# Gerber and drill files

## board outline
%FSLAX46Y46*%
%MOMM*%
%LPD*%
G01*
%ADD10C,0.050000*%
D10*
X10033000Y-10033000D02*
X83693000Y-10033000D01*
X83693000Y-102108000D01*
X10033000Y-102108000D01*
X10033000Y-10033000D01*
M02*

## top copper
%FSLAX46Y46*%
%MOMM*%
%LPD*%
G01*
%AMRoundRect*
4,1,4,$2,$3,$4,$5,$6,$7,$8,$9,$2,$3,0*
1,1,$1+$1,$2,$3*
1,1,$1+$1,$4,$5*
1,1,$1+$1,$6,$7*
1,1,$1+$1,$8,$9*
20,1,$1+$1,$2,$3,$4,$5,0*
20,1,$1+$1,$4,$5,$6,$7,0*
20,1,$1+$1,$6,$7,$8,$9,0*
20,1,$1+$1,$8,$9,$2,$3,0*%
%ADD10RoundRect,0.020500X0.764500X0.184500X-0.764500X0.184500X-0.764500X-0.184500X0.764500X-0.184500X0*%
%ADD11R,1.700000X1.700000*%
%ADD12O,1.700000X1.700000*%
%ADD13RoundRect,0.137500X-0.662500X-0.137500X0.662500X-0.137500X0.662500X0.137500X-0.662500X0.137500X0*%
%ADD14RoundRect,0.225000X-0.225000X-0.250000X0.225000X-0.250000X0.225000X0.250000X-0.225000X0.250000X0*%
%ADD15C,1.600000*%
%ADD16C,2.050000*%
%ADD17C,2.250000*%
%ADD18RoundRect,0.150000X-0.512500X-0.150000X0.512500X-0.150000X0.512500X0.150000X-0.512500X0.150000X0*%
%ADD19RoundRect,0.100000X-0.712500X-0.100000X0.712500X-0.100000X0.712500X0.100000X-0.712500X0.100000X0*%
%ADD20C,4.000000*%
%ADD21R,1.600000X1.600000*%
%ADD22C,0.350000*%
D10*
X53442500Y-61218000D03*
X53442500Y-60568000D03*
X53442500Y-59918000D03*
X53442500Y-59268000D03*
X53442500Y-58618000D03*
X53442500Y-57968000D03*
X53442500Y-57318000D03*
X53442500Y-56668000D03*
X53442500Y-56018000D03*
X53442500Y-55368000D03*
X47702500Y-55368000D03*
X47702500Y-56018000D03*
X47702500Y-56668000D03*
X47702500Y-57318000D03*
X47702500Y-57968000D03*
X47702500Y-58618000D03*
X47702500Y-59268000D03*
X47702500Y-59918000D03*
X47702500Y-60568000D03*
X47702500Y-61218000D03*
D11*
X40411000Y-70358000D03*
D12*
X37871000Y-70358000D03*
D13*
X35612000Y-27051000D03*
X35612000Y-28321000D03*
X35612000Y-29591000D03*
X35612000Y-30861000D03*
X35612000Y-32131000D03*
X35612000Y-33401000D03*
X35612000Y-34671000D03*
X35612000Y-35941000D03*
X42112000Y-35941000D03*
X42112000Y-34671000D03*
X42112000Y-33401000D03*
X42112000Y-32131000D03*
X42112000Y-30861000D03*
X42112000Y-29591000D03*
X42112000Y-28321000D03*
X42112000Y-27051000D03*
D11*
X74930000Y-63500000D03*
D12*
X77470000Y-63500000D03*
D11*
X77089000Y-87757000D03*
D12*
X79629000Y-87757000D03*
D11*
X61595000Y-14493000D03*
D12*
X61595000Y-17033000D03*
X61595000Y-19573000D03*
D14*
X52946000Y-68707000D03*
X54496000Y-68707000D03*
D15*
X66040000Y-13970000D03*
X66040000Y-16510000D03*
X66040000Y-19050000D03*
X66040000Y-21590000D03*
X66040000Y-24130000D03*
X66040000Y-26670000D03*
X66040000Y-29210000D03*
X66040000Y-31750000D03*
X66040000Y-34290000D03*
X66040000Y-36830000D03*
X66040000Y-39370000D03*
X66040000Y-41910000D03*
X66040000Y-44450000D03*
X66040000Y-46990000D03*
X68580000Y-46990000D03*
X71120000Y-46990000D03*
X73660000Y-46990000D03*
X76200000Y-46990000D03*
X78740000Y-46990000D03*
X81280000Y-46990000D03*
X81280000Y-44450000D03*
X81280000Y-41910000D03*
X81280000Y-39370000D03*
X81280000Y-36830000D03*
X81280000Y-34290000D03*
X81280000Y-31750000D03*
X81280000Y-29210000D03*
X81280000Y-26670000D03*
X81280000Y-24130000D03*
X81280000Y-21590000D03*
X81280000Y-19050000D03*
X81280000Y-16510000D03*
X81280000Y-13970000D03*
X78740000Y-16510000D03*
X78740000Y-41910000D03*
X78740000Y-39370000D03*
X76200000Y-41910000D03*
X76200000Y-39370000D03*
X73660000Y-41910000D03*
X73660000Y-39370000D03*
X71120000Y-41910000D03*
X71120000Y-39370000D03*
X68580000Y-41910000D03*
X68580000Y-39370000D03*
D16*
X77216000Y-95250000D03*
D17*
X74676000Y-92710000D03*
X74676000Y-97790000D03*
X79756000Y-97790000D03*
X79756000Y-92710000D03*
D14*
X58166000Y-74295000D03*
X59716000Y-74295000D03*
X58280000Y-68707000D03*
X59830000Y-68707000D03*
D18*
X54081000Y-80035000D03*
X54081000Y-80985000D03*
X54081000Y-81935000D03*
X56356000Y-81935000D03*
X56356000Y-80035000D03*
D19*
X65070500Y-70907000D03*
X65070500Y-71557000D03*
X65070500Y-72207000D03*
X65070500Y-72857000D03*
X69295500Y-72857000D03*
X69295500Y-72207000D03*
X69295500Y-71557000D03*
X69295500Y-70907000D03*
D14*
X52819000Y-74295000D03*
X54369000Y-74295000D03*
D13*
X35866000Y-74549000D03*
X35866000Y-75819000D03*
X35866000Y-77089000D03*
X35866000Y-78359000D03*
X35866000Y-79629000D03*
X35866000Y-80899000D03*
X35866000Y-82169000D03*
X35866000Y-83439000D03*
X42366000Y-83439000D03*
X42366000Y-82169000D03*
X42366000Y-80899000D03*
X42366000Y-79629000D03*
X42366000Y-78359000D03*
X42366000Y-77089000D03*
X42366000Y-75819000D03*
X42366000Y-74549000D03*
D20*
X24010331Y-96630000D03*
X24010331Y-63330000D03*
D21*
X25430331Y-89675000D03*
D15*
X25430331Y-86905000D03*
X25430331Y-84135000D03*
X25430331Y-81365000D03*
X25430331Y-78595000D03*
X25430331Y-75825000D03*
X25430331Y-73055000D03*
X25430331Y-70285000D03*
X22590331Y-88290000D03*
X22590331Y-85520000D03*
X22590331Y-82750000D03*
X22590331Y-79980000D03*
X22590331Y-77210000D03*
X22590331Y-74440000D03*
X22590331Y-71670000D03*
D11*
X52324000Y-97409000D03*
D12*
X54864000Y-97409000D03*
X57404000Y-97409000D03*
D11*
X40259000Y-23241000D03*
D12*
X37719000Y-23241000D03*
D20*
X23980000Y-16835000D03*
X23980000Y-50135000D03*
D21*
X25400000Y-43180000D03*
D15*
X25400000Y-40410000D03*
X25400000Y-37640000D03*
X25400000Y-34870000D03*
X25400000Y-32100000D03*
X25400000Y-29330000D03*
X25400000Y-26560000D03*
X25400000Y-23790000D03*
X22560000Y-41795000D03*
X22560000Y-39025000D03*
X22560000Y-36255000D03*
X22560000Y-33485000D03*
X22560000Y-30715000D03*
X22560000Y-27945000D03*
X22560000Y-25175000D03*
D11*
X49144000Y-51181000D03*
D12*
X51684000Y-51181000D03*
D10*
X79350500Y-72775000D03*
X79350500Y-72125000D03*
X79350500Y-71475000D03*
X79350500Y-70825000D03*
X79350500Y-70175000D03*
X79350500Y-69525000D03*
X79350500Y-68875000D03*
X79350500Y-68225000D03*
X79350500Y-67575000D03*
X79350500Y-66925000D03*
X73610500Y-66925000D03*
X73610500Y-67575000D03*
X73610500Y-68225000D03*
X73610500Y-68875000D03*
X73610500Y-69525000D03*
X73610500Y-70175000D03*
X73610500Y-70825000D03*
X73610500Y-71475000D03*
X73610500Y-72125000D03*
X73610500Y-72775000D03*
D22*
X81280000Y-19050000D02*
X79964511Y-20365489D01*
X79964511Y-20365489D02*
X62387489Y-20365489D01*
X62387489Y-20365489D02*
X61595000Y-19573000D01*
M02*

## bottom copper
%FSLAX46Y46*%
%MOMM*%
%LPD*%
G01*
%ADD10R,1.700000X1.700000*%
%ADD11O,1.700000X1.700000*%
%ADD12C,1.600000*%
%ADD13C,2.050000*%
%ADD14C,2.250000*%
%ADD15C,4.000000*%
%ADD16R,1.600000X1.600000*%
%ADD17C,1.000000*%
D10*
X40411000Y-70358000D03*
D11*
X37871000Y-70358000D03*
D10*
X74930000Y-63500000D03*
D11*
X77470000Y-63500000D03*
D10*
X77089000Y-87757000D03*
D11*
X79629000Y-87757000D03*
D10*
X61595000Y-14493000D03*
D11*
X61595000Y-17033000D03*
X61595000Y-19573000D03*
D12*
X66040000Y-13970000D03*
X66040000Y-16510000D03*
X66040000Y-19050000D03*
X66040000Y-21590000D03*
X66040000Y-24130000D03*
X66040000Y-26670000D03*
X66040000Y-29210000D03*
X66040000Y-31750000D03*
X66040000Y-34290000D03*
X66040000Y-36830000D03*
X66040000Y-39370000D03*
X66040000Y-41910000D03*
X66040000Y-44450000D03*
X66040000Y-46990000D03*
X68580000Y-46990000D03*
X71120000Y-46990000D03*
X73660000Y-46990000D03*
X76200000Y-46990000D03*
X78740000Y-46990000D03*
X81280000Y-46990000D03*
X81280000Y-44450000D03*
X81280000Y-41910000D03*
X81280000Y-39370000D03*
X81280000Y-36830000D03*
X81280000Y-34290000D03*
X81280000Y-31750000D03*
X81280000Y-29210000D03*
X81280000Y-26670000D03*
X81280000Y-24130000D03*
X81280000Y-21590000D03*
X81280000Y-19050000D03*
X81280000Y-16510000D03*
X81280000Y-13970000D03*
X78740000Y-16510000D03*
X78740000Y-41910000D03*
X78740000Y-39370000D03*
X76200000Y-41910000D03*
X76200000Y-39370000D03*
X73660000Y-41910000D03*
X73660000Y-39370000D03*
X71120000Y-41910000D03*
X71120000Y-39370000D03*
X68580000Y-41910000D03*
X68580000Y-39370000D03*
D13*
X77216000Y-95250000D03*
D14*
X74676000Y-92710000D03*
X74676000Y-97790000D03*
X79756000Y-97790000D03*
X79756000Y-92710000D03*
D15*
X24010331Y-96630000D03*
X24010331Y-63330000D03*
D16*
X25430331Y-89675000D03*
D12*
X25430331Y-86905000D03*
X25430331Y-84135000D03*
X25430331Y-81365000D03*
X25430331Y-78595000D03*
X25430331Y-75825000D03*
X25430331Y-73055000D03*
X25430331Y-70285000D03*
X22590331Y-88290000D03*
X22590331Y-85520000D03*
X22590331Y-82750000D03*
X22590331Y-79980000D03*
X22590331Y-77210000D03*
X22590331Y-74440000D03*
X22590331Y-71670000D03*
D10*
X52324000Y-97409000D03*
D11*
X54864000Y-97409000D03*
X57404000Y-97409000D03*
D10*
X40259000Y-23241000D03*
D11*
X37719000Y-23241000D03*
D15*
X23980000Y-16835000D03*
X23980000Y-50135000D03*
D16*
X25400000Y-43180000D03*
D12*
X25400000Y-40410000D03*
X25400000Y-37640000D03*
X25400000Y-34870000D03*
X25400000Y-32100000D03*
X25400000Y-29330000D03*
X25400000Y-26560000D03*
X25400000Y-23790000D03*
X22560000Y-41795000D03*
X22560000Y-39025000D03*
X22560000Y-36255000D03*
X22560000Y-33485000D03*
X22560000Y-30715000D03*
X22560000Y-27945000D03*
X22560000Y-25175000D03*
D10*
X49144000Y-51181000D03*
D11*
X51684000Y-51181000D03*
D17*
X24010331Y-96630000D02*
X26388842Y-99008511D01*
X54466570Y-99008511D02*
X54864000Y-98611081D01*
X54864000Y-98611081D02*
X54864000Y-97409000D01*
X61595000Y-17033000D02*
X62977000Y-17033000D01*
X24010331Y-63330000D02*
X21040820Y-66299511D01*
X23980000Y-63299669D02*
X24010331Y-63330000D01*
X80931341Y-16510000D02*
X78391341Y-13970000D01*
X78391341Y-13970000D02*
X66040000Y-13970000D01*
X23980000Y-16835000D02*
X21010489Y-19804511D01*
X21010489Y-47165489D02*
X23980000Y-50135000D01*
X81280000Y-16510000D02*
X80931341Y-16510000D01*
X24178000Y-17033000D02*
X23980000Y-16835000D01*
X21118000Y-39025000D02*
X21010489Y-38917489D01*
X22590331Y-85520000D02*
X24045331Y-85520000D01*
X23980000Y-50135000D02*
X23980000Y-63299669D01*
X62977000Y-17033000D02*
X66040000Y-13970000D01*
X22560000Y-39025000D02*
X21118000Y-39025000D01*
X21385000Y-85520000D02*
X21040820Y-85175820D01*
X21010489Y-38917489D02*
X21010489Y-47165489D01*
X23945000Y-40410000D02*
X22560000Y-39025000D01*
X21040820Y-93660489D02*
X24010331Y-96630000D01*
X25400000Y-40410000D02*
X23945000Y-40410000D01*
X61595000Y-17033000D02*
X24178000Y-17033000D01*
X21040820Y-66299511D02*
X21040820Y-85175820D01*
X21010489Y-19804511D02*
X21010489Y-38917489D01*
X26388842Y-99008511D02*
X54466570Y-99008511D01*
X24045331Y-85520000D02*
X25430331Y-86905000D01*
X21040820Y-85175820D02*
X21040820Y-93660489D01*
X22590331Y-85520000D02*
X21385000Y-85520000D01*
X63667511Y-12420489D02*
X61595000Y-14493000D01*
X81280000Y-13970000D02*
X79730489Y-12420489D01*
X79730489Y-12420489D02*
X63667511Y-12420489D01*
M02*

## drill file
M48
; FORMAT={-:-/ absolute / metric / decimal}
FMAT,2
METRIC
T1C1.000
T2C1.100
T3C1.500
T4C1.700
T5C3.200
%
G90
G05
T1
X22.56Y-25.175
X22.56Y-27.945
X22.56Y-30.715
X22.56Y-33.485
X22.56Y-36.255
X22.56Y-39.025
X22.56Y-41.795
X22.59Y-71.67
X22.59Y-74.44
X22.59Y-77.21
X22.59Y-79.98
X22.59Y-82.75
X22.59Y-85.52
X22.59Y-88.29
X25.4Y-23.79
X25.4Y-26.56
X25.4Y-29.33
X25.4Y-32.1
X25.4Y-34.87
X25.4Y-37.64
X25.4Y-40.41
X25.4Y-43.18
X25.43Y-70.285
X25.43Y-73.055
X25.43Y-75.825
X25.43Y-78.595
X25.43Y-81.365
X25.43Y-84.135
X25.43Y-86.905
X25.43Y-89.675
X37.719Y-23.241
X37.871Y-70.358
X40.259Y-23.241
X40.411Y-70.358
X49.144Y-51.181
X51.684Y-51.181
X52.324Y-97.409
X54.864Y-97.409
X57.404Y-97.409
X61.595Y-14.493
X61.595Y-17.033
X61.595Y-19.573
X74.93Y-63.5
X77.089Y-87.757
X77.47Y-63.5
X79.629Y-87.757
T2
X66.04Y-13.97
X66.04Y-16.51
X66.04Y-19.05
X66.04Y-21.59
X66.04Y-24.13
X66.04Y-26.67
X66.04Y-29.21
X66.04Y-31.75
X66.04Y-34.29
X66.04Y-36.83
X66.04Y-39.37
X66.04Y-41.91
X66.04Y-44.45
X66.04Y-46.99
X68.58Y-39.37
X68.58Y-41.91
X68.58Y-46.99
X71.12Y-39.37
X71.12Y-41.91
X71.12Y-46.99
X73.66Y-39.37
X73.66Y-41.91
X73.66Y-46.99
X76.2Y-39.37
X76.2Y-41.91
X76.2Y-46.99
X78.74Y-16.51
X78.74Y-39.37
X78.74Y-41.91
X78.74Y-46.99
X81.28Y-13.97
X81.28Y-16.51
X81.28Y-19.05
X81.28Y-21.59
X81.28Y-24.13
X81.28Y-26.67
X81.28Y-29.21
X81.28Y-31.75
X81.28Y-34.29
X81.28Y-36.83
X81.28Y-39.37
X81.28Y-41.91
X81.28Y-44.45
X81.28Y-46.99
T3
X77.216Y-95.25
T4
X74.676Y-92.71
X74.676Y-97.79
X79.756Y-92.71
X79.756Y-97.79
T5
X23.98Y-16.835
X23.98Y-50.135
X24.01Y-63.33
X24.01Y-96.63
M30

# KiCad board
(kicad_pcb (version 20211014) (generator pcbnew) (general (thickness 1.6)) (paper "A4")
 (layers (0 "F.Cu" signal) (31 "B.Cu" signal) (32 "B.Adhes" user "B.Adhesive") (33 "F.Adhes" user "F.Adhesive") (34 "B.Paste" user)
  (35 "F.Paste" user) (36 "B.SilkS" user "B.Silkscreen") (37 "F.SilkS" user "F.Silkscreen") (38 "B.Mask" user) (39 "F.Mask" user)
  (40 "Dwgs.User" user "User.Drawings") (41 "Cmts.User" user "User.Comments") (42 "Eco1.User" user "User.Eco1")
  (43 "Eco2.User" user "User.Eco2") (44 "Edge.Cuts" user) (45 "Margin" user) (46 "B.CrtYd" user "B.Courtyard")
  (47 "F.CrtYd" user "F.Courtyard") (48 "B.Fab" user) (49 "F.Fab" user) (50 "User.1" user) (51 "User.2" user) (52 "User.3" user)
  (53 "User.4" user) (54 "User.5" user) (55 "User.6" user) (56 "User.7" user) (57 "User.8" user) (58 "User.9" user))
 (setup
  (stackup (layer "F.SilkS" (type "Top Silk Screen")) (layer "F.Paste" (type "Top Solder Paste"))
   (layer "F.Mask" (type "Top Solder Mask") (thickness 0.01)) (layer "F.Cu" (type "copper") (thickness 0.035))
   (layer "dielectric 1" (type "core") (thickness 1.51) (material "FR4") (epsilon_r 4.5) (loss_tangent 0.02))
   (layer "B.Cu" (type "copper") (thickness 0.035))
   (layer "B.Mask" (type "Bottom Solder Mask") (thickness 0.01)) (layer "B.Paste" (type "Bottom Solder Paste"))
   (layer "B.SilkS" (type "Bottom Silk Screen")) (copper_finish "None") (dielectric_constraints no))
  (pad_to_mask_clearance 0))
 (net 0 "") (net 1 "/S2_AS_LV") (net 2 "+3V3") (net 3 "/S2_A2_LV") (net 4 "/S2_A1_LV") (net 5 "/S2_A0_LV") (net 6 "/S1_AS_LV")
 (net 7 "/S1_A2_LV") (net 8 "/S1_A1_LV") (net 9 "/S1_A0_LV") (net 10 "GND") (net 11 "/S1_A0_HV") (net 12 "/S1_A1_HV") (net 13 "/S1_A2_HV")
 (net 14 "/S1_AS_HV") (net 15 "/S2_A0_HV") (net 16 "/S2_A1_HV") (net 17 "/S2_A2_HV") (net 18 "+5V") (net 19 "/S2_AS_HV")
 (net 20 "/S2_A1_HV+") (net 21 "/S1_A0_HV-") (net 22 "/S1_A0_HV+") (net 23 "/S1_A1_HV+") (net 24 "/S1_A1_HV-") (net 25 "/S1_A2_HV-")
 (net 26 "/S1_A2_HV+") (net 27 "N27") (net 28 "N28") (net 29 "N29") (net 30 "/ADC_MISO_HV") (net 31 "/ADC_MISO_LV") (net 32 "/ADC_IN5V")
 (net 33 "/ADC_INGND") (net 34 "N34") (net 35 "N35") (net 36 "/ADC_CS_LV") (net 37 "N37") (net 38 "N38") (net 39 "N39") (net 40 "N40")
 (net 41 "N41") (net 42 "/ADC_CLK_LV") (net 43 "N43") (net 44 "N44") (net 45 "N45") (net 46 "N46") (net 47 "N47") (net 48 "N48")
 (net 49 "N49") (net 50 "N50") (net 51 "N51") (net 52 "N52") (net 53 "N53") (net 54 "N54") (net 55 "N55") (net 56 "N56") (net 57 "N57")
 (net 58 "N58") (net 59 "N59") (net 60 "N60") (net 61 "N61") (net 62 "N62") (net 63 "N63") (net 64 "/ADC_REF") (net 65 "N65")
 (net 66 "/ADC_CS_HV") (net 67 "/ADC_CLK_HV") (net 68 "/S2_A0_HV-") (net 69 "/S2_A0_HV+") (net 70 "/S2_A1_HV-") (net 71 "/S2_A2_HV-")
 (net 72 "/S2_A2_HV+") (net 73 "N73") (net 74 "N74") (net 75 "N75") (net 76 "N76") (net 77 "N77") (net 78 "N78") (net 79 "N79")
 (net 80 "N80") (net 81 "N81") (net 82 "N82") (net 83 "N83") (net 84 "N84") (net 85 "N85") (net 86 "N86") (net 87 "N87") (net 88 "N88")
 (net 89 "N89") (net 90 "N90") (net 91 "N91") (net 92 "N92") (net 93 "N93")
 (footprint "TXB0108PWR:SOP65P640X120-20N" (layer "F.Cu") (at 50.5725 58.293 180)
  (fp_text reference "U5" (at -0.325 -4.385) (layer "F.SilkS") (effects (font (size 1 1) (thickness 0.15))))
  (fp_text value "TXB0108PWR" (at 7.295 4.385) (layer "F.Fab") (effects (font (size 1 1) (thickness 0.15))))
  (pad "1" smd roundrect locked (at -2.87 -2.925 180) (size 1.57 0.41) (layers "F.Cu" "F.Paste" "F.Mask") (roundrect_rratio 0.05)
   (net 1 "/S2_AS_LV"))
  (pad "2" smd roundrect locked (at -2.87 -2.275 180) (size 1.57 0.41) (layers "F.Cu" "F.Paste" "F.Mask") (roundrect_rratio 0.05)
   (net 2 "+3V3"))
  (pad "3" smd roundrect locked (at -2.87 -1.625 180) (size 1.57 0.41) (layers "F.Cu" "F.Paste" "F.Mask") (roundrect_rratio 0.05)
   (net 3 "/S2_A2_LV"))
  (pad "4" smd roundrect locked (at -2.87 -0.975 180) (size 1.57 0.41) (layers "F.Cu" "F.Paste" "F.Mask") (roundrect_rratio 0.05)
   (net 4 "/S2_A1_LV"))
  (pad "5" smd roundrect locked (at -2.87 -0.325 180) (size 1.57 0.41) (layers "F.Cu" "F.Paste" "F.Mask") (roundrect_rratio 0.05)
   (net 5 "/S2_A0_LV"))
  (pad "6" smd roundrect locked (at -2.87 0.325 180) (size 1.57 0.41) (layers "F.Cu" "F.Paste" "F.Mask") (roundrect_rratio 0.05)
   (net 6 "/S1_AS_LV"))
  (pad "7" smd roundrect locked (at -2.87 0.975 180) (size 1.57 0.41) (layers "F.Cu" "F.Paste" "F.Mask") (roundrect_rratio 0.05)
   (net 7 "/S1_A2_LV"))
  (pad "8" smd roundrect locked (at -2.87 1.625 180) (size 1.57 0.41) (layers "F.Cu" "F.Paste" "F.Mask") (roundrect_rratio 0.05)
   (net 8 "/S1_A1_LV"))
  (pad "9" smd roundrect locked (at -2.87 2.275 180) (size 1.57 0.41) (layers "F.Cu" "F.Paste" "F.Mask") (roundrect_rratio 0.05)
   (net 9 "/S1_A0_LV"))
  (pad "10" smd roundrect locked (at -2.87 2.925 180) (size 1.57 0.41) (layers "F.Cu" "F.Paste" "F.Mask") (roundrect_rratio 0.05)
   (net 2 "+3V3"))
  (pad "11" smd roundrect locked (at 2.87 2.925 180) (size 1.57 0.41) (layers "F.Cu" "F.Paste" "F.Mask") (roundrect_rratio 0.05)
   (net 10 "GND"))
  (pad "12" smd roundrect locked (at 2.87 2.275 180) (size 1.57 0.41) (layers "F.Cu" "F.Paste" "F.Mask") (roundrect_rratio 0.05)
   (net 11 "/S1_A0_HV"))
  (pad "13" smd roundrect locked (at 2.87 1.625 180) (size 1.57 0.41) (layers "F.Cu" "F.Paste" "F.Mask") (roundrect_rratio 0.05)
   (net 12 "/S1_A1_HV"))
  (pad "14" smd roundrect locked (at 2.87 0.975 180) (size 1.57 0.41) (layers "F.Cu" "F.Paste" "F.Mask") (roundrect_rratio 0.05)
   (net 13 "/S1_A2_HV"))
  (pad "15" smd roundrect locked (at 2.87 0.325 180) (size 1.57 0.41) (layers "F.Cu" "F.Paste" "F.Mask") (roundrect_rratio 0.05)
   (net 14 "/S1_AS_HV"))
  (pad "16" smd roundrect locked (at 2.87 -0.325 180) (size 1.57 0.41) (layers "F.Cu" "F.Paste" "F.Mask") (roundrect_rratio 0.05)
   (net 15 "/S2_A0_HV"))
  (pad "17" smd roundrect locked (at 2.87 -0.975 180) (size 1.57 0.41) (layers "F.Cu" "F.Paste" "F.Mask") (roundrect_rratio 0.05)
   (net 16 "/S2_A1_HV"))
  (pad "18" smd roundrect locked (at 2.87 -1.625 180) (size 1.57 0.41) (layers "F.Cu" "F.Paste" "F.Mask") (roundrect_rratio 0.05)
   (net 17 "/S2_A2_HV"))
  (pad "19" smd roundrect locked (at 2.87 -2.275 180) (size 1.57 0.41) (layers "F.Cu" "F.Paste" "F.Mask") (roundrect_rratio 0.05)
   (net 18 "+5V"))
  (pad "20" smd roundrect locked (at 2.87 -2.925 180) (size 1.57 0.41) (layers "F.Cu" "F.Paste" "F.Mask") (roundrect_rratio 0.05)
   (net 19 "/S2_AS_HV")))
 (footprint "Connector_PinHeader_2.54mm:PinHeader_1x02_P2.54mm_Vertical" (layer "F.Cu") (at 40.411 70.358 -90)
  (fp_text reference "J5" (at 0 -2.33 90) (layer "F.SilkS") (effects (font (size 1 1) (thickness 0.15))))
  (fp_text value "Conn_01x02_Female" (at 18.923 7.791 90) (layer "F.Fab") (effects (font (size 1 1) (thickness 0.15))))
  (pad "1" thru_hole rect (at 0 0 270) (size 1.7 1.7) (drill 1) (layers *.Cu *.Mask) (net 18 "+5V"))
  (pad "2" thru_hole oval (at 0 2.54 270) (size 1.7 1.7) (drill 1) (layers *.Cu *.Mask) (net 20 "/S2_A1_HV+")))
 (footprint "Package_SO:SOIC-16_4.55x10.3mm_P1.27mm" (layer "F.Cu") (at 38.862 31.496)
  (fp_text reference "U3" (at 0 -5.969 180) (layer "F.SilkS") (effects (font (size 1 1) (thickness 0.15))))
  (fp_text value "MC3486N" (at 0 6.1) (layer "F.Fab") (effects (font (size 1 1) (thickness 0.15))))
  (pad "1" smd roundrect (at -3.25 -4.445) (size 1.6 0.55) (layers "F.Cu" "F.Paste" "F.Mask") (roundrect_rratio 0.25) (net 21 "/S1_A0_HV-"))
  (pad "2" smd roundrect (at -3.25 -3.175) (size 1.6 0.55) (layers "F.Cu" "F.Paste" "F.Mask") (roundrect_rratio 0.25) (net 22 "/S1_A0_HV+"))
  (pad "3" smd roundrect (at -3.25 -1.905) (size 1.6 0.55) (layers "F.Cu" "F.Paste" "F.Mask") (roundrect_rratio 0.25) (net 11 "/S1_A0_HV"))
  (pad "4" smd roundrect (at -3.25 -0.635) (size 1.6 0.55) (layers "F.Cu" "F.Paste" "F.Mask") (roundrect_rratio 0.25) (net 18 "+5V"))
  (pad "5" smd roundrect (at -3.25 0.635) (size 1.6 0.55) (layers "F.Cu" "F.Paste" "F.Mask") (roundrect_rratio 0.25) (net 12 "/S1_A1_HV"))
  (pad "6" smd roundrect (at -3.25 1.905) (size 1.6 0.55) (layers "F.Cu" "F.Paste" "F.Mask") (roundrect_rratio 0.25) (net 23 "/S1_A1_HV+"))
  (pad "7" smd roundrect (at -3.25 3.175) (size 1.6 0.55) (layers "F.Cu" "F.Paste" "F.Mask") (roundrect_rratio 0.25) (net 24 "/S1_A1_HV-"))
  (pad "8" smd roundrect (at -3.25 4.445) (size 1.6 0.55) (layers "F.Cu" "F.Paste" "F.Mask") (roundrect_rratio 0.25) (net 10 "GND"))
  (pad "9" smd roundrect (at 3.25 4.445) (size 1.6 0.55) (layers "F.Cu" "F.Paste" "F.Mask") (roundrect_rratio 0.25) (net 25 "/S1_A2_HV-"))
  (pad "10" smd roundrect (at 3.25 3.175) (size 1.6 0.55) (layers "F.Cu" "F.Paste" "F.Mask") (roundrect_rratio 0.25) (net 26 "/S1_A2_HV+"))
  (pad "11" smd roundrect (at 3.25 1.905) (size 1.6 0.55) (layers "F.Cu" "F.Paste" "F.Mask") (roundrect_rratio 0.25) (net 13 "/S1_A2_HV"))
  (pad "12" smd roundrect (at 3.25 0.635) (size 1.6 0.55) (layers "F.Cu" "F.Paste" "F.Mask") (roundrect_rratio 0.25) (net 18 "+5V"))
  (pad "13" smd roundrect (at 3.25 -0.635) (size 1.6 0.55) (layers "F.Cu" "F.Paste" "F.Mask") (roundrect_rratio 0.25) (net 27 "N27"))
  (pad "14" smd roundrect (at 3.25 -1.905) (size 1.6 0.55) (layers "F.Cu" "F.Paste" "F.Mask") (roundrect_rratio 0.25) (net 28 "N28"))
  (pad "15" smd roundrect (at 3.25 -3.175) (size 1.6 0.55) (layers "F.Cu" "F.Paste" "F.Mask") (roundrect_rratio 0.25) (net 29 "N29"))
  (pad "16" smd roundrect (at 3.25 -4.445) (size 1.6 0.55) (layers "F.Cu" "F.Paste" "F.Mask") (roundrect_rratio 0.25) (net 18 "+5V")))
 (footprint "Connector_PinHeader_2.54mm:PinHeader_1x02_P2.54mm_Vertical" (layer "F.Cu") (at 74.93 63.5 90)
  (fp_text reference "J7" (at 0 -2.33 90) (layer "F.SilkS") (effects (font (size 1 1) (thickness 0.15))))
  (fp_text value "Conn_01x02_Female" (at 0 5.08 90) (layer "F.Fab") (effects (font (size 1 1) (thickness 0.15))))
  (pad "1" thru_hole rect (at 0 0 90) (size 1.7 1.7) (drill 1) (layers *.Cu *.Mask) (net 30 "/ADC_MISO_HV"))
  (pad "2" thru_hole oval (at 0 2.54 90) (size 1.7 1.7) (drill 1) (layers *.Cu *.Mask) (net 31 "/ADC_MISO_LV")))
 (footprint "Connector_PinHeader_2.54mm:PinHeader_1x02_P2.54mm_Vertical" (layer "F.Cu") (at 77.089 87.757 90)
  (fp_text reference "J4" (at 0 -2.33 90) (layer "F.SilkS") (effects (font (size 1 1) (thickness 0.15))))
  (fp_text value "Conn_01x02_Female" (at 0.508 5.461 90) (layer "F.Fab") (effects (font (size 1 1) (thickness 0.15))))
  (pad "1" thru_hole rect (at 0 0 90) (size 1.7 1.7) (drill 1) (layers *.Cu *.Mask) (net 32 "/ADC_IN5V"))
  (pad "2" thru_hole oval (at 0 2.54 90) (size 1.7 1.7) (drill 1) (layers *.Cu *.Mask) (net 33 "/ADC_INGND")))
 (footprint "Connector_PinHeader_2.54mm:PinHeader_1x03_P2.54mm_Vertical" (layer "F.Cu") (at 61.595 14.493)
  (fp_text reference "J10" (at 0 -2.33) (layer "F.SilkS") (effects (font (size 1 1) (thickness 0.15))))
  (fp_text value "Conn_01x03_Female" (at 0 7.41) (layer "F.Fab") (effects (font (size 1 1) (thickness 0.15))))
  (pad "1" thru_hole rect (at 0 0) (size 1.7 1.7) (drill 1) (layers *.Cu *.Mask) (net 18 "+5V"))
  (pad "2" thru_hole oval (at 0 2.54) (size 1.7 1.7) (drill 1) (layers *.Cu *.Mask) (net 10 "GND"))
  (pad "3" thru_hole oval (at 0 5.08) (size 1.7 1.7) (drill 1) (layers *.Cu *.Mask) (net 2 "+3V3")))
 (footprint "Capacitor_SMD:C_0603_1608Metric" (layer "F.Cu") (at 53.721 68.707)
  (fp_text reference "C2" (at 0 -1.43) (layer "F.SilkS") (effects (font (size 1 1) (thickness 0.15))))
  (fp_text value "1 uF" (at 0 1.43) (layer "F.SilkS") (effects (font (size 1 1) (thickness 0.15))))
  (pad "1" smd roundrect (at -0.775 0) (size 0.9 0.95) (layers "F.Cu" "F.Paste" "F.Mask") (roundrect_rratio 0.25) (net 18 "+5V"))
  (pad "2" smd roundrect (at 0.775 0) (size 0.9 0.95) (layers "F.Cu" "F.Paste" "F.Mask") (roundrect_rratio 0.25) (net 10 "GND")))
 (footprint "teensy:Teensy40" (layer "F.Cu") (at 73.66 30.48 -90)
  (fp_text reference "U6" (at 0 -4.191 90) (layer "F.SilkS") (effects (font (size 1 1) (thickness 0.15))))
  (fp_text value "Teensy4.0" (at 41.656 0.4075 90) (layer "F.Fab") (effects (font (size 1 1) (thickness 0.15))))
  (pad "1" thru_hole circle locked (at -16.51 7.62 270) (size 1.6 1.6) (drill 1.1) (layers *.Cu *.Mask) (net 10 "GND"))
  (pad "2" thru_hole circle locked (at -13.97 7.62 270) (size 1.6 1.6) (drill 1.1) (layers *.Cu *.Mask) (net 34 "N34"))
  (pad "3" thru_hole circle locked (at -11.43 7.62 270) (size 1.6 1.6) (drill 1.1) (layers *.Cu *.Mask) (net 8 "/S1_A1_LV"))
  (pad "4" thru_hole circle locked (at -8.89 7.62 270) (size 1.6 1.6) (drill 1.1) (layers *.Cu *.Mask) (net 7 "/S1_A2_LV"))
  (pad "5" thru_hole circle locked (at -6.35 7.62 270) (size 1.6 1.6) (drill 1.1) (layers *.Cu *.Mask) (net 4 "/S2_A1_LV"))
  (pad "6" thru_hole circle locked (at -3.81 7.62 270) (size 1.6 1.6) (drill 1.1) (layers *.Cu *.Mask) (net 3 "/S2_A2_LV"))
  (pad "7" thru_hole circle locked (at -1.27 7.62 270) (size 1.6 1.6) (drill 1.1) (layers *.Cu *.Mask) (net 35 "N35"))
  (pad "8" thru_hole circle locked (at 1.27 7.62 270) (size 1.6 1.6) (drill 1.1) (layers *.Cu *.Mask) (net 9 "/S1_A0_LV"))
  (pad "9" thru_hole circle locked (at 3.81 7.62 270) (size 1.6 1.6) (drill 1.1) (layers *.Cu *.Mask) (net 5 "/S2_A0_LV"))
  (pad "10" thru_hole circle locked (at 6.35 7.62 270) (size 1.6 1.6) (drill 1.1) (layers *.Cu *.Mask) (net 6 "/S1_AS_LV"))
  (pad "11" thru_hole circle locked (at 8.89 7.62 270) (size 1.6 1.6) (drill 1.1) (layers *.Cu *.Mask) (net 1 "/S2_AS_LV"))
  (pad "12" thru_hole circle locked (at 11.43 7.62 270) (size 1.6 1.6) (drill 1.1) (layers *.Cu *.Mask) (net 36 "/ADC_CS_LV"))
  (pad "13" thru_hole circle locked (at 13.97 7.62 270) (size 1.6 1.6) (drill 1.1) (layers *.Cu *.Mask) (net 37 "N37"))
  (pad "14" thru_hole circle locked (at 16.51 7.62 270) (size 1.6 1.6) (drill 1.1) (layers *.Cu *.Mask) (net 31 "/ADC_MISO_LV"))
  (pad "15" thru_hole circle locked (at 16.51 5.08 270) (size 1.6 1.6) (drill 1.1) (layers *.Cu *.Mask) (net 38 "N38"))
  (pad "16" thru_hole circle locked (at 16.51 2.54 270) (size 1.6 1.6) (drill 1.1) (layers *.Cu *.Mask) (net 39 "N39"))
  (pad "17" thru_hole circle locked (at 16.51 0 270) (size 1.6 1.6) (drill 1.1) (layers *.Cu *.Mask) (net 10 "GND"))
  (pad "18" thru_hole circle locked (at 16.51 -2.54 270) (size 1.6 1.6) (drill 1.1) (layers *.Cu *.Mask) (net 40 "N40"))
  (pad "19" thru_hole circle locked (at 16.51 -5.08 270) (size 1.6 1.6) (drill 1.1) (layers *.Cu *.Mask) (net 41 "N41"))
  (pad "20" thru_hole circle locked (at 16.51 -7.62 270) (size 1.6 1.6) (drill 1.1) (layers *.Cu *.Mask) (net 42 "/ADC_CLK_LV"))
  (pad "21" thru_hole circle locked (at 13.97 -7.62 270) (size 1.6 1.6) (drill 1.1) (layers *.Cu *.Mask) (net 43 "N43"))
  (pad "22" thru_hole circle locked (at 11.43 -7.62 270) (size 1.6 1.6) (drill 1.1) (layers *.Cu *.Mask) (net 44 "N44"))
  (pad "23" thru_hole circle locked (at 8.89 -7.62 270) (size 1.6 1.6) (drill 1.1) (layers *.Cu *.Mask) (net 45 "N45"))
  (pad "24" thru_hole circle locked (at 6.35 -7.62 270) (size 1.6 1.6) (drill 1.1) (layers *.Cu *.Mask) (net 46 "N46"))
  (pad "25" thru_hole circle locked (at 3.81 -7.62 270) (size 1.6 1.6) (drill 1.1) (layers *.Cu *.Mask) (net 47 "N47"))
  (pad "26" thru_hole circle locked (at 1.27 -7.62 270) (size 1.6 1.6) (drill 1.1) (layers *.Cu *.Mask) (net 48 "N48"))
  (pad "27" thru_hole circle locked (at -1.27 -7.62 270) (size 1.6 1.6) (drill 1.1) (layers *.Cu *.Mask) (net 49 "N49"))
  (pad "28" thru_hole circle locked (at -3.81 -7.62 270) (size 1.6 1.6) (drill 1.1) (layers *.Cu *.Mask) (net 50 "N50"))
  (pad "29" thru_hole circle locked (at -6.35 -7.62 270) (size 1.6 1.6) (drill 1.1) (layers *.Cu *.Mask) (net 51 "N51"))
  (pad "30" thru_hole circle locked (at -8.89 -7.62 270) (size 1.6 1.6) (drill 1.1) (layers *.Cu *.Mask) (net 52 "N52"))
  (pad "31" thru_hole circle locked (at -11.43 -7.62 270) (size 1.6 1.6) (drill 1.1) (layers *.Cu *.Mask) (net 2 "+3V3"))
  (pad "32" thru_hole circle locked (at -13.97 -7.62 270) (size 1.6 1.6) (drill 1.1) (layers *.Cu *.Mask) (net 10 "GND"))
  (pad "33" thru_hole circle locked (at -16.51 -7.62 270) (size 1.6 1.6) (drill 1.1) (layers *.Cu *.Mask) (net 18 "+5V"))
  (pad "34" thru_hole circle locked (at -13.97 -5.08 270) (size 1.6 1.6) (drill 1.1) (layers *.Cu *.Mask) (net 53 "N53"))
  (pad "35" thru_hole circle locked (at 11.43 -5.08 270) (size 1.6 1.6) (drill 1.1) (layers *.Cu *.Mask) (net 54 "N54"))
  (pad "36" thru_hole circle locked (at 8.89 -5.08 270) (size 1.6 1.6) (drill 1.1) (layers *.Cu *.Mask) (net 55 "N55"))
  (pad "37" thru_hole circle locked (at 11.43 -2.54 270) (size 1.6 1.6) (drill 1.1) (layers *.Cu *.Mask) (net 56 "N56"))
  (pad "38" thru_hole circle locked (at 8.89 -2.54 270) (size 1.6 1.6) (drill 1.1) (layers *.Cu *.Mask) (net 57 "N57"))
  (pad "39" thru_hole circle locked (at 11.43 0 270) (size 1.6 1.6) (drill 1.1) (layers *.Cu *.Mask) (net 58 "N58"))
  (pad "40" thru_hole circle locked (at 8.89 0 270) (size 1.6 1.6) (drill 1.1) (layers *.Cu *.Mask) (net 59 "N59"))
  (pad "41" thru_hole circle locked (at 11.43 2.54 270) (size 1.6 1.6) (drill 1.1) (layers *.Cu *.Mask) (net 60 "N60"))
  (pad "42" thru_hole circle locked (at 8.89 2.54 270) (size 1.6 1.6) (drill 1.1) (layers *.Cu *.Mask) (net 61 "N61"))
  (pad "43" thru_hole circle locked (at 11.43 5.08 270) (size 1.6 1.6) (drill 1.1) (layers *.Cu *.Mask) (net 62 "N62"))
  (pad "44" thru_hole circle locked (at 8.89 5.08 270) (size 1.6 1.6) (drill 1.1) (layers *.Cu *.Mask) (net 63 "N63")))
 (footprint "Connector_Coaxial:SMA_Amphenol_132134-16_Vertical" (layer "F.Cu") (at 77.216 95.25)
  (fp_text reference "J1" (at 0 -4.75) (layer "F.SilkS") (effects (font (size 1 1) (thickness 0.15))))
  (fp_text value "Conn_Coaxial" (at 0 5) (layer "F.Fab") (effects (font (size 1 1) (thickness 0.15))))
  (pad "1" thru_hole circle (at 0 0) (size 2.05 2.05) (drill 1.5) (layers *.Cu *.Mask) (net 32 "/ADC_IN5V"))
  (pad "2" thru_hole circle (at -2.54 -2.54) (size 2.25 2.25) (drill 1.7) (layers *.Cu *.Mask) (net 33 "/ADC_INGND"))
  (pad "2" thru_hole circle (at -2.54 2.54) (size 2.25 2.25) (drill 1.7) (layers *.Cu *.Mask) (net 33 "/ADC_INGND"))
  (pad "2" thru_hole circle (at 2.54 2.54) (size 2.25 2.25) (drill 1.7) (layers *.Cu *.Mask) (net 33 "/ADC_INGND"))
  (pad "2" thru_hole circle (at 2.54 -2.54) (size 2.25 2.25) (drill 1.7) (layers *.Cu *.Mask) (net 33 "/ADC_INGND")))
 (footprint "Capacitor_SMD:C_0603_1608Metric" (layer "F.Cu") (at 58.941 74.295)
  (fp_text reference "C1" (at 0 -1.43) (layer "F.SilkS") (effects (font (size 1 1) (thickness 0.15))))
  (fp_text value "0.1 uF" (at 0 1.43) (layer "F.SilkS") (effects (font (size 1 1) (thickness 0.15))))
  (pad "1" smd roundrect (at -0.775 0) (size 0.9 0.95) (layers "F.Cu" "F.Paste" "F.Mask") (roundrect_rratio 0.25) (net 18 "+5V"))
  (pad "2" smd roundrect (at 0.775 0) (size 0.9 0.95) (layers "F.Cu" "F.Paste" "F.Mask") (roundrect_rratio 0.25) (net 10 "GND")))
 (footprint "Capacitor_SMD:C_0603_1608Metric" (layer "F.Cu") (at 59.055 68.707)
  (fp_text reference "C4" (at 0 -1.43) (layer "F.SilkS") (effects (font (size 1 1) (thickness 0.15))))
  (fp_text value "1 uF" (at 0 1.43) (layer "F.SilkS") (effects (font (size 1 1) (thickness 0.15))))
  (pad "1" smd roundrect (at -0.775 0) (size 0.9 0.95) (layers "F.Cu" "F.Paste" "F.Mask") (roundrect_rratio 0.25) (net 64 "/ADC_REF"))
  (pad "2" smd roundrect (at 0.775 0) (size 0.9 0.95) (layers "F.Cu" "F.Paste" "F.Mask") (roundrect_rratio 0.25) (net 10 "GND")))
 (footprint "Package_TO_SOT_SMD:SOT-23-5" (layer "F.Cu") (at 55.2185 80.985)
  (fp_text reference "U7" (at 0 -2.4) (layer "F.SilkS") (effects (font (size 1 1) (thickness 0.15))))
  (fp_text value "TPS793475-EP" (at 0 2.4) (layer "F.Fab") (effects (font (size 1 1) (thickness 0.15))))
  (pad "1" smd roundrect (at -1.1375 -0.95) (size 1.325 0.6) (layers "F.Cu" "F.Paste" "F.Mask") (roundrect_rratio 0.25) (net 18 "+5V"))
  (pad "2" smd roundrect (at -1.1375 0) (size 1.325 0.6) (layers "F.Cu" "F.Paste" "F.Mask") (roundrect_rratio 0.25) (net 10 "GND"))
  (pad "3" smd roundrect (at -1.1375 0.95) (size 1.325 0.6) (layers "F.Cu" "F.Paste" "F.Mask") (roundrect_rratio 0.25) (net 10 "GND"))
  (pad "4" smd roundrect (at 1.1375 0.95) (size 1.325 0.6) (layers "F.Cu" "F.Paste" "F.Mask") (roundrect_rratio 0.25) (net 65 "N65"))
  (pad "5" smd roundrect (at 1.1375 -0.95) (size 1.325 0.6) (layers "F.Cu" "F.Paste" "F.Mask") (roundrect_rratio 0.25) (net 64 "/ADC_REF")))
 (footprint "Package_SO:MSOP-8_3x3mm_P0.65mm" (layer "F.Cu") (at 67.183 71.882)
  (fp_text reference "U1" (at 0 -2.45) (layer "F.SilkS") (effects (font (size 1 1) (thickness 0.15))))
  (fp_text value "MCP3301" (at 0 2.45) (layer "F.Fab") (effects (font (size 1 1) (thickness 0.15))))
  (pad "1" smd roundrect (at -2.1125 -0.975) (size 1.625 0.4) (layers "F.Cu" "F.Paste" "F.Mask") (roundrect_rratio 0.25) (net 64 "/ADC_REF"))
  (pad "2" smd roundrect (at -2.1125 -0.325) (size 1.625 0.4) (layers "F.Cu" "F.Paste" "F.Mask") (roundrect_rratio 0.25)
   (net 32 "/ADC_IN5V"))
  (pad "3" smd roundrect (at -2.1125 0.325) (size 1.625 0.4) (layers "F.Cu" "F.Paste" "F.Mask") (roundrect_rratio 0.25)
   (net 33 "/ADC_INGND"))
  (pad "4" smd roundrect (at -2.1125 0.975) (size 1.625 0.4) (layers "F.Cu" "F.Paste" "F.Mask") (roundrect_rratio 0.25) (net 10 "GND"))
  (pad "5" smd roundrect (at 2.1125 0.975) (size 1.625 0.4) (layers "F.Cu" "F.Paste" "F.Mask") (roundrect_rratio 0.25) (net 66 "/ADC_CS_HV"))
  (pad "6" smd roundrect (at 2.1125 0.325) (size 1.625 0.4) (layers "F.Cu" "F.Paste" "F.Mask") (roundrect_rratio 0.25)
   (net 30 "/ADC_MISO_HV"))
  (pad "7" smd roundrect (at 2.1125 -0.325) (size 1.625 0.4) (layers "F.Cu" "F.Paste" "F.Mask") (roundrect_rratio 0.25)
   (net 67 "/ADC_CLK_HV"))
  (pad "8" smd roundrect (at 2.1125 -0.975) (size 1.625 0.4) (layers "F.Cu" "F.Paste" "F.Mask") (roundrect_rratio 0.25) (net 18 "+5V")))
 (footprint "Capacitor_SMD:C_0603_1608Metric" (layer "F.Cu") (at 53.594 74.295)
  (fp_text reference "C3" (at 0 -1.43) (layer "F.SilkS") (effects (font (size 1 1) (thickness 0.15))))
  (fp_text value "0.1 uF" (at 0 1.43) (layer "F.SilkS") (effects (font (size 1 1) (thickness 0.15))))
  (pad "1" smd roundrect (at -0.775 0) (size 0.9 0.95) (layers "F.Cu" "F.Paste" "F.Mask") (roundrect_rratio 0.25) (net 65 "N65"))
  (pad "2" smd roundrect (at 0.775 0) (size 0.9 0.95) (layers "F.Cu" "F.Paste" "F.Mask") (roundrect_rratio 0.25) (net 10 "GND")))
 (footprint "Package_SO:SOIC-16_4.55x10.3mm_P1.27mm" (layer "F.Cu") (at 39.116 78.994)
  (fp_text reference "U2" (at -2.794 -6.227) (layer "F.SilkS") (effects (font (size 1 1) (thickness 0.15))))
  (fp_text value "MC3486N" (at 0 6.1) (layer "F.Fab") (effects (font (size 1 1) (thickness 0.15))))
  (pad "1" smd roundrect (at -3.25 -4.445) (size 1.6 0.55) (layers "F.Cu" "F.Paste" "F.Mask") (roundrect_rratio 0.25) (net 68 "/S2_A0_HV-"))
  (pad "2" smd roundrect (at -3.25 -3.175) (size 1.6 0.55) (layers "F.Cu" "F.Paste" "F.Mask") (roundrect_rratio 0.25) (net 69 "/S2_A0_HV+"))
  (pad "3" smd roundrect (at -3.25 -1.905) (size 1.6 0.55) (layers "F.Cu" "F.Paste" "F.Mask") (roundrect_rratio 0.25) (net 15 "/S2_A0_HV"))
  (pad "4" smd roundrect (at -3.25 -0.635) (size 1.6 0.55) (layers "F.Cu" "F.Paste" "F.Mask") (roundrect_rratio 0.25) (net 18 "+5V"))
  (pad "5" smd roundrect (at -3.25 0.635) (size 1.6 0.55) (layers "F.Cu" "F.Paste" "F.Mask") (roundrect_rratio 0.25) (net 16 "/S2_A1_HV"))
  (pad "6" smd roundrect (at -3.25 1.905) (size 1.6 0.55) (layers "F.Cu" "F.Paste" "F.Mask") (roundrect_rratio 0.25) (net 20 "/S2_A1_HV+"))
  (pad "7" smd roundrect (at -3.25 3.175) (size 1.6 0.55) (layers "F.Cu" "F.Paste" "F.Mask") (roundrect_rratio 0.25) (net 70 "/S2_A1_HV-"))
  (pad "8" smd roundrect (at -3.25 4.445) (size 1.6 0.55) (layers "F.Cu" "F.Paste" "F.Mask") (roundrect_rratio 0.25) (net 10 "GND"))
  (pad "9" smd roundrect (at 3.25 4.445) (size 1.6 0.55) (layers "F.Cu" "F.Paste" "F.Mask") (roundrect_rratio 0.25) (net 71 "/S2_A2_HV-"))
  (pad "10" smd roundrect (at 3.25 3.175) (size 1.6 0.55) (layers "F.Cu" "F.Paste" "F.Mask") (roundrect_rratio 0.25) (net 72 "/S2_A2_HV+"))
  (pad "11" smd roundrect (at 3.25 1.905) (size 1.6 0.55) (layers "F.Cu" "F.Paste" "F.Mask") (roundrect_rratio 0.25) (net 17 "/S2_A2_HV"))
  (pad "12" smd roundrect (at 3.25 0.635) (size 1.6 0.55) (layers "F.Cu" "F.Paste" "F.Mask") (roundrect_rratio 0.25) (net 18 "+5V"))
  (pad "13" smd roundrect (at 3.25 -0.635) (size 1.6 0.55) (layers "F.Cu" "F.Paste" "F.Mask") (roundrect_rratio 0.25) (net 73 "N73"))
  (pad "14" smd roundrect (at 3.25 -1.905) (size 1.6 0.55) (layers "F.Cu" "F.Paste" "F.Mask") (roundrect_rratio 0.25) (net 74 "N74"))
  (pad "15" smd roundrect (at 3.25 -3.175) (size 1.6 0.55) (layers "F.Cu" "F.Paste" "F.Mask") (roundrect_rratio 0.25) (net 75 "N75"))
  (pad "16" smd roundrect (at 3.25 -4.445) (size 1.6 0.55) (layers "F.Cu" "F.Paste" "F.Mask") (roundrect_rratio 0.25) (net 18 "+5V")))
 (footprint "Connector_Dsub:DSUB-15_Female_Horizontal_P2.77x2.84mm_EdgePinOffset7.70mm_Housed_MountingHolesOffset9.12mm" (layer "F.Cu")
  (at 25.430331 89.675 -90)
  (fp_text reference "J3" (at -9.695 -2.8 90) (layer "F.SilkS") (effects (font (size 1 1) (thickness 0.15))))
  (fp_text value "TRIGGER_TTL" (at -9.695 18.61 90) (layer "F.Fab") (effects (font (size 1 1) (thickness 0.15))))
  (pad "0" thru_hole circle (at 6.955 1.42 270) (size 4 4) (drill 3.2) (layers *.Cu *.Mask) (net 10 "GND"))
  (pad "0" thru_hole circle (at -26.345 1.42 270) (size 4 4) (drill 3.2) (layers *.Cu *.Mask) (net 10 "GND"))
  (pad "1" thru_hole rect (at 0 0 270) (size 1.6 1.6) (drill 1) (layers *.Cu *.Mask) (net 20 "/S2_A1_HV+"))
  (pad "2" thru_hole circle (at -2.77 0 270) (size 1.6 1.6) (drill 1) (layers *.Cu *.Mask) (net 10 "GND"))
  (pad "3" thru_hole circle (at -5.54 0 270) (size 1.6 1.6) (drill 1) (layers *.Cu *.Mask) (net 72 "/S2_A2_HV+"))
  (pad "4" thru_hole circle (at -8.31 0 270) (size 1.6 1.6) (drill 1) (layers *.Cu *.Mask) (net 18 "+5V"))
  (pad "5" thru_hole circle (at -11.08 0 270) (size 1.6 1.6) (drill 1) (layers *.Cu *.Mask) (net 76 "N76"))
  (pad "6" thru_hole circle (at -13.85 0 270) (size 1.6 1.6) (drill 1) (layers *.Cu *.Mask) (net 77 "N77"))
  (pad "7" thru_hole circle (at -16.62 0 270) (size 1.6 1.6) (drill 1) (layers *.Cu *.Mask) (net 68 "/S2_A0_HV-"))
  (pad "8" thru_hole circle (at -19.39 0 270) (size 1.6 1.6) (drill 1) (layers *.Cu *.Mask) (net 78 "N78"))
  (pad "9" thru_hole circle (at -1.385 2.84 270) (size 1.6 1.6) (drill 1) (layers *.Cu *.Mask) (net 70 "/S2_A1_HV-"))
  (pad "10" thru_hole circle (at -4.155 2.84 270) (size 1.6 1.6) (drill 1) (layers *.Cu *.Mask) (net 10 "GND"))
  (pad "11" thru_hole circle (at -6.925 2.84 270) (size 1.6 1.6) (drill 1) (layers *.Cu *.Mask) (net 71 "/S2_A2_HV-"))
  (pad "12" thru_hole circle (at -9.695 2.84 270) (size 1.6 1.6) (drill 1) (layers *.Cu *.Mask) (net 18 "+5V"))
  (pad "13" thru_hole circle (at -12.465 2.84 270) (size 1.6 1.6) (drill 1) (layers *.Cu *.Mask) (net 19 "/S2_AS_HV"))
  (pad "14" thru_hole circle (at -15.235 2.84 270) (size 1.6 1.6) (drill 1) (layers *.Cu *.Mask) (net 69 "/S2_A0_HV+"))
  (pad "15" thru_hole circle (at -18.005 2.84 270) (size 1.6 1.6) (drill 1) (layers *.Cu *.Mask) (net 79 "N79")))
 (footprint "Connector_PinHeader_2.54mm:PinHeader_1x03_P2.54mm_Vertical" (layer "F.Cu") (at 52.324 97.409 90)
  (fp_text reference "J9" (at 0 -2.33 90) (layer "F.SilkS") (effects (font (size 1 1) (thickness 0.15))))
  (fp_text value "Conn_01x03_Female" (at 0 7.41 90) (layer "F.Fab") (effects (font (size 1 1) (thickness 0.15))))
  (pad "1" thru_hole rect (at 0 0 90) (size 1.7 1.7) (drill 1) (layers *.Cu *.Mask) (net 18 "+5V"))
  (pad "2" thru_hole oval (at 0 2.54 90) (size 1.7 1.7) (drill 1) (layers *.Cu *.Mask) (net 10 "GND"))
  (pad "3" thru_hole oval (at 0 5.08 90) (size 1.7 1.7) (drill 1) (layers *.Cu *.Mask) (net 64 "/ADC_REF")))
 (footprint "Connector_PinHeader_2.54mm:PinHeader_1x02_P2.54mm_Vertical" (layer "F.Cu") (at 40.259 23.241 -90)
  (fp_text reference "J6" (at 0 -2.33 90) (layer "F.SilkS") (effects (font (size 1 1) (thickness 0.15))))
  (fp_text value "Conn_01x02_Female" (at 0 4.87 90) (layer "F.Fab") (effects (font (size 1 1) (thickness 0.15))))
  (pad "1" thru_hole rect (at 0 0 270) (size 1.7 1.7) (drill 1) (layers *.Cu *.Mask) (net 18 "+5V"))
  (pad "2" thru_hole oval (at 0 2.54 270) (size 1.7 1.7) (drill 1) (layers *.Cu *.Mask) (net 23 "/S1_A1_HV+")))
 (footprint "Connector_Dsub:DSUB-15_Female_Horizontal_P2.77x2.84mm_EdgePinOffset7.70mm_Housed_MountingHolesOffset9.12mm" (layer "F.Cu")
  (at 25.4 43.18 -90)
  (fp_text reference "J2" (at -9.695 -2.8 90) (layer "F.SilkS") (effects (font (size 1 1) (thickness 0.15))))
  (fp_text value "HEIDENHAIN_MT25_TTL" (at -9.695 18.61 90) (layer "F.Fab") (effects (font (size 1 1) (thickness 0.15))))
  (pad "0" thru_hole circle (at -26.345 1.42 270) (size 4 4) (drill 3.2) (layers *.Cu *.Mask) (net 10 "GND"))
  (pad "0" thru_hole circle (at 6.955 1.42 270) (size 4 4) (drill 3.2) (layers *.Cu *.Mask) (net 10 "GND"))
  (pad "1" thru_hole rect (at 0 0 270) (size 1.6 1.6) (drill 1) (layers *.Cu *.Mask) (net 23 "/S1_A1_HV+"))
  (pad "2" thru_hole circle (at -2.77 0 270) (size 1.6 1.6) (drill 1) (layers *.Cu *.Mask) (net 10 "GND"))
  (pad "3" thru_hole circle (at -5.54 0 270) (size 1.6 1.6) (drill 1) (layers *.Cu *.Mask) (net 26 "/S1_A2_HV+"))
  (pad "4" thru_hole circle (at -8.31 0 270) (size 1.6 1.6) (drill 1) (layers *.Cu *.Mask) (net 18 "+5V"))
  (pad "5" thru_hole circle (at -11.08 0 270) (size 1.6 1.6) (drill 1) (layers *.Cu *.Mask) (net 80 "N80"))
  (pad "6" thru_hole circle (at -13.85 0 270) (size 1.6 1.6) (drill 1) (layers *.Cu *.Mask) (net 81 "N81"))
  (pad "7" thru_hole circle (at -16.62 0 270) (size 1.6 1.6) (drill 1) (layers *.Cu *.Mask) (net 21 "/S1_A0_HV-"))
  (pad "8" thru_hole circle (at -19.39 0 270) (size 1.6 1.6) (drill 1) (layers *.Cu *.Mask) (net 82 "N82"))
  (pad "9" thru_hole circle (at -1.385 2.84 270) (size 1.6 1.6) (drill 1) (layers *.Cu *.Mask) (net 24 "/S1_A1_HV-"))
  (pad "10" thru_hole circle (at -4.155 2.84 270) (size 1.6 1.6) (drill 1) (layers *.Cu *.Mask) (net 10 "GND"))
  (pad "11" thru_hole circle (at -6.925 2.84 270) (size 1.6 1.6) (drill 1) (layers *.Cu *.Mask) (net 25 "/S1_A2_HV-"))
  (pad "12" thru_hole circle (at -9.695 2.84 270) (size 1.6 1.6) (drill 1) (layers *.Cu *.Mask) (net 18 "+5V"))
  (pad "13" thru_hole circle (at -12.465 2.84 270) (size 1.6 1.6) (drill 1) (layers *.Cu *.Mask) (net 14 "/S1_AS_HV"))
  (pad "14" thru_hole circle (at -15.235 2.84 270) (size 1.6 1.6) (drill 1) (layers *.Cu *.Mask) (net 22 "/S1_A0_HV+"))
  (pad "15" thru_hole circle (at -18.005 2.84 270) (size 1.6 1.6) (drill 1) (layers *.Cu *.Mask) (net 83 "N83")))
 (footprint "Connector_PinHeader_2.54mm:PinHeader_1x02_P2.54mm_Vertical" (layer "F.Cu") (at 49.144 51.181 90)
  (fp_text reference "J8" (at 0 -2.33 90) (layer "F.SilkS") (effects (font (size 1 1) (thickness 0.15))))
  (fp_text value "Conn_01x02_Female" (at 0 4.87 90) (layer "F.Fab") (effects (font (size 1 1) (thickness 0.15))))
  (pad "1" thru_hole rect (at 0 0 90) (size 1.7 1.7) (drill 1) (layers *.Cu *.Mask) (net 12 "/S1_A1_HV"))
  (pad "2" thru_hole oval (at 0 2.54 90) (size 1.7 1.7) (drill 1) (layers *.Cu *.Mask) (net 8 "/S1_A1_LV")))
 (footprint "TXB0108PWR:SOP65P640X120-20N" (layer "F.Cu") (at 76.4805 69.85 180)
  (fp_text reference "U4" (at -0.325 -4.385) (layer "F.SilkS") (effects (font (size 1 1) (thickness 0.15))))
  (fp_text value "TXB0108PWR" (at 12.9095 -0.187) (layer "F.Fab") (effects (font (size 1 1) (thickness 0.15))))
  (pad "1" smd roundrect locked (at -2.87 -2.925 180) (size 1.57 0.41) (layers "F.Cu" "F.Paste" "F.Mask") (roundrect_rratio 0.05)
   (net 42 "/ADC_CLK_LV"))
  (pad "2" smd roundrect locked (at -2.87 -2.275 180) (size 1.57 0.41) (layers "F.Cu" "F.Paste" "F.Mask") (roundrect_rratio 0.05)
   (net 2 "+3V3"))
  (pad "3" smd roundrect locked (at -2.87 -1.625 180) (size 1.57 0.41) (layers "F.Cu" "F.Paste" "F.Mask") (roundrect_rratio 0.05)
   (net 31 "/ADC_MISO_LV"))
  (pad "4" smd roundrect locked (at -2.87 -0.975 180) (size 1.57 0.41) (layers "F.Cu" "F.Paste" "F.Mask") (roundrect_rratio 0.05)
   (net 36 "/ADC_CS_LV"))
  (pad "5" smd roundrect locked (at -2.87 -0.325 180) (size 1.57 0.41) (layers "F.Cu" "F.Paste" "F.Mask") (roundrect_rratio 0.05)
   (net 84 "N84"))
  (pad "6" smd roundrect locked (at -2.87 0.325 180) (size 1.57 0.41) (layers "F.Cu" "F.Paste" "F.Mask") (roundrect_rratio 0.05)
   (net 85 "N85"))
  (pad "7" smd roundrect locked (at -2.87 0.975 180) (size 1.57 0.41) (layers "F.Cu" "F.Paste" "F.Mask") (roundrect_rratio 0.05)
   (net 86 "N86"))
  (pad "8" smd roundrect locked (at -2.87 1.625 180) (size 1.57 0.41) (layers "F.Cu" "F.Paste" "F.Mask") (roundrect_rratio 0.05)
   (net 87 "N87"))
  (pad "9" smd roundrect locked (at -2.87 2.275 180) (size 1.57 0.41) (layers "F.Cu" "F.Paste" "F.Mask") (roundrect_rratio 0.05)
   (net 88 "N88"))
  (pad "10" smd roundrect locked (at -2.87 2.925 180) (size 1.57 0.41) (layers "F.Cu" "F.Paste" "F.Mask") (roundrect_rratio 0.05)
   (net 2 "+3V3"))
  (pad "11" smd roundrect locked (at 2.87 2.925 180) (size 1.57 0.41) (layers "F.Cu" "F.Paste" "F.Mask") (roundrect_rratio 0.05)
   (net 10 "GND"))
  (pad "12" smd roundrect locked (at 2.87 2.275 180) (size 1.57 0.41) (layers "F.Cu" "F.Paste" "F.Mask") (roundrect_rratio 0.05)
   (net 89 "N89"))
  (pad "13" smd roundrect locked (at 2.87 1.625 180) (size 1.57 0.41) (layers "F.Cu" "F.Paste" "F.Mask") (roundrect_rratio 0.05)
   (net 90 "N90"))
  (pad "14" smd roundrect locked (at 2.87 0.975 180) (size 1.57 0.41) (layers "F.Cu" "F.Paste" "F.Mask") (roundrect_rratio 0.05)
   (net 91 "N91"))
  (pad "15" smd roundrect locked (at 2.87 0.325 180) (size 1.57 0.41) (layers "F.Cu" "F.Paste" "F.Mask") (roundrect_rratio 0.05)
   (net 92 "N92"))
  (pad "16" smd roundrect locked (at 2.87 -0.325 180) (size 1.57 0.41) (layers "F.Cu" "F.Paste" "F.Mask") (roundrect_rratio 0.05)
   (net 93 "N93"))
  (pad "17" smd roundrect locked (at 2.87 -0.975 180) (size 1.57 0.41) (layers "F.Cu" "F.Paste" "F.Mask") (roundrect_rratio 0.05)
   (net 66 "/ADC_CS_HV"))
  (pad "18" smd roundrect locked (at 2.87 -1.625 180) (size 1.57 0.41) (layers "F.Cu" "F.Paste" "F.Mask") (roundrect_rratio 0.05)
   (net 30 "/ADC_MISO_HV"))
  (pad "19" smd roundrect locked (at 2.87 -2.275 180) (size 1.57 0.41) (layers "F.Cu" "F.Paste" "F.Mask") (roundrect_rratio 0.05)
   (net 18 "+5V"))
  (pad "20" smd roundrect locked (at 2.87 -2.925 180) (size 1.57 0.41) (layers "F.Cu" "F.Paste" "F.Mask") (roundrect_rratio 0.05)
   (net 67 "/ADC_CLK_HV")))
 (gr_rect (start 10.033 10.033) (end 83.693 102.108) (layer "Edge.Cuts") (width 0.05) (fill none))
 (segment (start 24.010331 96.63) (end 26.388842 99.008511) (width 1) (layer "B.Cu") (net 10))
 (segment (start 54.46657 99.008511) (end 54.864 98.611081) (width 1) (layer "B.Cu") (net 10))
 (segment (start 54.864 98.611081) (end 54.864 97.409) (width 1) (layer "B.Cu") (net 10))
 (segment (start 61.595 17.033) (end 62.977 17.033) (width 1) (layer "B.Cu") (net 10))
 (segment (start 24.010331 63.33) (end 21.04082 66.299511) (width 1) (layer "B.Cu") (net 10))
 (segment (start 23.98 63.299669) (end 24.010331 63.33) (width 1) (layer "B.Cu") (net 10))
 (segment (start 80.931341 16.51) (end 78.391341 13.97) (width 1) (layer "B.Cu") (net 10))
 (segment (start 78.391341 13.97) (end 66.04 13.97) (width 1) (layer "B.Cu") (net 10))
 (segment (start 23.98 16.835) (end 21.010489 19.804511) (width 1) (layer "B.Cu") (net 10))
 (segment (start 21.010489 47.165489) (end 23.98 50.135) (width 1) (layer "B.Cu") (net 10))
 (segment (start 81.28 16.51) (end 80.931341 16.51) (width 1) (layer "B.Cu") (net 10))
 (segment (start 24.178 17.033) (end 23.98 16.835) (width 1) (layer "B.Cu") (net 10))
 (segment (start 21.118 39.025) (end 21.010489 38.917489) (width 1) (layer "B.Cu") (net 10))
 (segment (start 22.590331 85.52) (end 24.045331 85.52) (width 1) (layer "B.Cu") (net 10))
 (segment (start 23.98 50.135) (end 23.98 63.299669) (width 1) (layer "B.Cu") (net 10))
 (segment (start 62.977 17.033) (end 66.04 13.97) (width 1) (layer "B.Cu") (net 10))
 (segment (start 22.56 39.025) (end 21.118 39.025) (width 1) (layer "B.Cu") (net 10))
 (segment (start 21.385 85.52) (end 21.04082 85.17582) (width 1) (layer "B.Cu") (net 10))
 (segment (start 21.010489 38.917489) (end 21.010489 47.165489) (width 1) (layer "B.Cu") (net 10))
 (segment (start 23.945 40.41) (end 22.56 39.025) (width 1) (layer "B.Cu") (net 10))
 (segment (start 21.04082 93.660489) (end 24.010331 96.63) (width 1) (layer "B.Cu") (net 10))
 (segment (start 25.4 40.41) (end 23.945 40.41) (width 1) (layer "B.Cu") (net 10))
 (segment (start 61.595 17.033) (end 24.178 17.033) (width 1) (layer "B.Cu") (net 10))
 (segment (start 21.04082 66.299511) (end 21.04082 85.17582) (width 1) (layer "B.Cu") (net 10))
 (segment (start 21.010489 19.804511) (end 21.010489 38.917489) (width 1) (layer "B.Cu") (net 10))
 (segment (start 26.388842 99.008511) (end 54.46657 99.008511) (width 1) (layer "B.Cu") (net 10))
 (segment (start 24.045331 85.52) (end 25.430331 86.905) (width 1) (layer "B.Cu") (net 10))
 (segment (start 21.04082 85.17582) (end 21.04082 93.660489) (width 1) (layer "B.Cu") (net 10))
 (segment (start 22.590331 85.52) (end 21.385 85.52) (width 1) (layer "B.Cu") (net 10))
 (segment (start 81.28 19.05) (end 79.964511 20.365489) (width 0.35) (layer "F.Cu") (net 2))
 (segment (start 79.964511 20.365489) (end 62.387489 20.365489) (width 0.35) (layer "F.Cu") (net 2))
 (segment (start 62.387489 20.365489) (end 61.595 19.573) (width 0.35) (layer "F.Cu") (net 2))
 (segment (start 63.667511 12.420489) (end 61.595 14.493) (width 1) (layer "B.Cu") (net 18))
 (segment (start 81.28 13.97) (end 79.730489 12.420489) (width 1) (layer "B.Cu") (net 18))
 (segment (start 79.730489 12.420489) (end 63.667511 12.420489) (width 1) (layer "B.Cu") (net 18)))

